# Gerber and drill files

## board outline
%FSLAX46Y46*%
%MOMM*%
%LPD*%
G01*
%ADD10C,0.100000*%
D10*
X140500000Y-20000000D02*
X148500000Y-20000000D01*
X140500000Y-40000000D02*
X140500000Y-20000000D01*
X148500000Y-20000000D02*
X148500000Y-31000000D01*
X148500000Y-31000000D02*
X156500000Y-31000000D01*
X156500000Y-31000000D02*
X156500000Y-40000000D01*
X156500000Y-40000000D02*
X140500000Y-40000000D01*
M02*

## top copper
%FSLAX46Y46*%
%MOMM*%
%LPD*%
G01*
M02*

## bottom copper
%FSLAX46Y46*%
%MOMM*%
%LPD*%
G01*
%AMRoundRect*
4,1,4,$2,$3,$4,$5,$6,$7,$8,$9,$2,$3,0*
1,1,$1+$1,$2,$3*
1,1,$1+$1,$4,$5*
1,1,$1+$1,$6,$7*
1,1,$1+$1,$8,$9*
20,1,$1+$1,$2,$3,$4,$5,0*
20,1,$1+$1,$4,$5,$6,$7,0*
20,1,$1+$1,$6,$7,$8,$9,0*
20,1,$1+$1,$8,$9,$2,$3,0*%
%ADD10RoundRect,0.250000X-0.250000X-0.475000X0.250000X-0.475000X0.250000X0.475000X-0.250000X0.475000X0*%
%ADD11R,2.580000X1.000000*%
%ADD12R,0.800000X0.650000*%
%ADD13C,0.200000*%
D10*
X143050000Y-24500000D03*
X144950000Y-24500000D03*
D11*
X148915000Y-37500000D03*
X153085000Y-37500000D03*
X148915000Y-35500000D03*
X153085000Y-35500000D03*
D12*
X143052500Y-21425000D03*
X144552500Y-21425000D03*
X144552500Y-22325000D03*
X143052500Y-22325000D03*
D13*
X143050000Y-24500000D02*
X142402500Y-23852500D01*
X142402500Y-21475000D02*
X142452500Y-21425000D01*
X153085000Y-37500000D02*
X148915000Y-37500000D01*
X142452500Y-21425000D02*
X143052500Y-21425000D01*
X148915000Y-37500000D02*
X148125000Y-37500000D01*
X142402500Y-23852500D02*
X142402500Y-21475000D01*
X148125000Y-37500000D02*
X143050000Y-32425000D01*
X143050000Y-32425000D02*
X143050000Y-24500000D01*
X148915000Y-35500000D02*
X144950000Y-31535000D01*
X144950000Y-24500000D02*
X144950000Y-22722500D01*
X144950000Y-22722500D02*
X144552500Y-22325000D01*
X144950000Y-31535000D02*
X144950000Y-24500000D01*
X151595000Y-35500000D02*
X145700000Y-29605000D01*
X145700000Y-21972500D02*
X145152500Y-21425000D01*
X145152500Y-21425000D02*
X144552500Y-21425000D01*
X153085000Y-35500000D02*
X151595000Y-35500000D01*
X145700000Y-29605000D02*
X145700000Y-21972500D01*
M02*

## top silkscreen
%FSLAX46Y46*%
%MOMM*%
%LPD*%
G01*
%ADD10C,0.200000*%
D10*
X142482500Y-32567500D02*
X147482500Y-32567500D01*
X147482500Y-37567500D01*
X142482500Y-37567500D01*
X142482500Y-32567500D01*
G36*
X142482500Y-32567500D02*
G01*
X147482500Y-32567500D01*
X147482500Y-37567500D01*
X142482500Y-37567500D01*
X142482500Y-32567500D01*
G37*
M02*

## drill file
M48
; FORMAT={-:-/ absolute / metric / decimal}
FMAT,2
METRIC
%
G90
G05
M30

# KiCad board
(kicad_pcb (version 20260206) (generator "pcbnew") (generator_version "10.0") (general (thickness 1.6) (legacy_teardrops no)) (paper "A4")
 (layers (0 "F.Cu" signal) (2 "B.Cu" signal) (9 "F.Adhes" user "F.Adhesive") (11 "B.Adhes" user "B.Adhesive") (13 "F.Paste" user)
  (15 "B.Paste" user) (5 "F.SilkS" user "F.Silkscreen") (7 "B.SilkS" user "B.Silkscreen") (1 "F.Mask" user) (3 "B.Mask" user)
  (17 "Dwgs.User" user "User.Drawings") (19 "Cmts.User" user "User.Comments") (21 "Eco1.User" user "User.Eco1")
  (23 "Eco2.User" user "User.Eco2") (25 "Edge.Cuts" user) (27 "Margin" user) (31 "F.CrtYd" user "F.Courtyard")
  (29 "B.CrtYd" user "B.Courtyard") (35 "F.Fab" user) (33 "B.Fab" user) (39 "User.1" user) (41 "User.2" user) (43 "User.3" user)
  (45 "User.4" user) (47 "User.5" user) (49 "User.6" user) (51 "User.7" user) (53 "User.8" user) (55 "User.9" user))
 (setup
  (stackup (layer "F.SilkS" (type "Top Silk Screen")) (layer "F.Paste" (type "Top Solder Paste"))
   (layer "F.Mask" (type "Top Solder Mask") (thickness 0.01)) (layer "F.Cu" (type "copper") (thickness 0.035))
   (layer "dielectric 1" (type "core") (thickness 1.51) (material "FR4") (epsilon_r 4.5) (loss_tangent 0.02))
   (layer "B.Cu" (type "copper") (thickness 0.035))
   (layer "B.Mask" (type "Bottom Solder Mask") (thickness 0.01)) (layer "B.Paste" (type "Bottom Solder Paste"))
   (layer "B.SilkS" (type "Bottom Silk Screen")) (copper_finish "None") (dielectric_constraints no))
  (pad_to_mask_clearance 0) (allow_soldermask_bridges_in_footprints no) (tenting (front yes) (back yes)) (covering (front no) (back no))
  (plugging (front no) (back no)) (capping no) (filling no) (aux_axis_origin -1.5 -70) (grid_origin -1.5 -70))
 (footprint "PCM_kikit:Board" (layer "F.Cu") (at 140.5 20)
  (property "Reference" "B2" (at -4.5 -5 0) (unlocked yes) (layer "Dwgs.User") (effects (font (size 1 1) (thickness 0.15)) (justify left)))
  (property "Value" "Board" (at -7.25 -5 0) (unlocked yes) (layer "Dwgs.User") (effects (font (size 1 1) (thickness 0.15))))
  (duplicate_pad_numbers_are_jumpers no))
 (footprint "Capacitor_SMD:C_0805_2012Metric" (layer "B.Cu") (at 144 24.5)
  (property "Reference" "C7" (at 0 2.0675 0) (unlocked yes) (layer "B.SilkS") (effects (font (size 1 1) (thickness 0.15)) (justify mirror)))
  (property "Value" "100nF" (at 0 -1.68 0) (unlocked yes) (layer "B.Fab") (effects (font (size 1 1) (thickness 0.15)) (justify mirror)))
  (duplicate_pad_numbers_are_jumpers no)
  (pad "1" smd roundrect (at -0.95 0) (size 1 1.45) (layers "B.Cu" "B.Mask" "B.Paste") (roundrect_rratio 0.25) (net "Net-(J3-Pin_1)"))
  (pad "2" smd roundrect (at 0.95 0) (size 1 1.45) (layers "B.Cu" "B.Mask" "B.Paste") (roundrect_rratio 0.25) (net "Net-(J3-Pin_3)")))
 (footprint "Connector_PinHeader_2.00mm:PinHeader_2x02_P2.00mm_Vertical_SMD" (layer "B.Cu") (at 151 36.5)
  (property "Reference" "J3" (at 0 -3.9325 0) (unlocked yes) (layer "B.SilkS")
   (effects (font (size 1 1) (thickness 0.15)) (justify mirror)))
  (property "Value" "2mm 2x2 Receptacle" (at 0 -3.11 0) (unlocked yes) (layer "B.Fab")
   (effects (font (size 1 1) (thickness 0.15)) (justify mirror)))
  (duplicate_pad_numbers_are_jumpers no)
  (pad "1" smd rect (at -2.085 1) (size 2.58 1) (layers "B.Cu" "B.Mask" "B.Paste") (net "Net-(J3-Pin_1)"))
  (pad "2" smd rect (at 2.085 1) (size 2.58 1) (layers "B.Cu" "B.Mask" "B.Paste") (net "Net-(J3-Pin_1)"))
  (pad "3" smd rect (at -2.085 -1) (size 2.58 1) (layers "B.Cu" "B.Mask" "B.Paste") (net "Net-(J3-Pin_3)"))
  (pad "4" smd rect (at 2.085 -1) (size 2.58 1) (layers "B.Cu" "B.Mask" "B.Paste") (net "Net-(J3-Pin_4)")))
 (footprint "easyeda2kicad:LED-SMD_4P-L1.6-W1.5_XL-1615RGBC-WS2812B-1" (layer "B.Cu") (at 143.8025 21.875)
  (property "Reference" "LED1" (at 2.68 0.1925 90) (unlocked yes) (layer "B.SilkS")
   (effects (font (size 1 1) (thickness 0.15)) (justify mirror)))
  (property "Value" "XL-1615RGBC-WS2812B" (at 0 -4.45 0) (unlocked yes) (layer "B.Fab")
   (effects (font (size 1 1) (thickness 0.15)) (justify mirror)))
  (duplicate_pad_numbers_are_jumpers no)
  (pad "1" smd rect (at -0.75 -0.45 180) (size 0.8 0.65) (layers "B.Cu" "B.Mask" "B.Paste") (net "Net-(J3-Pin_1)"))
  (pad "2" smd rect (at 0.75 -0.45 180) (size 0.8 0.65) (layers "B.Cu" "B.Mask" "B.Paste") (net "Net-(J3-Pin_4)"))
  (pad "3" smd rect (at 0.75 0.45 180) (size 0.8 0.65) (layers "B.Cu" "B.Mask" "B.Paste") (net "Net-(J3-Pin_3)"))
  (pad "4" smd rect (at -0.75 0.45 180) (size 0.8 0.65) (layers "B.Cu" "B.Mask" "B.Paste") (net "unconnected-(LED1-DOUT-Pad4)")))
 (gr_rect (start 142.4825 32.5675) (end 147.4825 37.5675) (stroke (width 0.2) (type solid)) (fill yes) (layer "F.SilkS"))
 (gr_line (start 140.5 20) (end 148.5 20) (stroke (width 0.1) (type default)) (layer "Edge.Cuts"))
 (gr_line (start 140.5 40) (end 140.5 20) (stroke (width 0.1) (type default)) (layer "Edge.Cuts"))
 (gr_line (start 148.5 20) (end 148.5 31) (stroke (width 0.1) (type default)) (layer "Edge.Cuts"))
 (gr_line (start 148.5 31) (end 156.5 31) (stroke (width 0.1) (type default)) (layer "Edge.Cuts"))
 (gr_line (start 156.5 31) (end 156.5 40) (stroke (width 0.1) (type default)) (layer "Edge.Cuts"))
 (gr_line (start 156.5 40) (end 140.5 40) (stroke (width 0.1) (type default)) (layer "Edge.Cuts"))
 (segment (start 143.05 24.5) (end 142.4025 23.8525) (width 0.2) (layer "B.Cu") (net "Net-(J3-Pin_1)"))
 (segment (start 142.4025 21.475) (end 142.4525 21.425) (width 0.2) (layer "B.Cu") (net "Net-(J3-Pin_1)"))
 (segment (start 153.085 37.5) (end 148.915 37.5) (width 0.2) (layer "B.Cu") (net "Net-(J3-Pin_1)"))
 (segment (start 142.4525 21.425) (end 143.0525 21.425) (width 0.2) (layer "B.Cu") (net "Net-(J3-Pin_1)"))
 (segment (start 148.915 37.5) (end 148.125 37.5) (width 0.2) (layer "B.Cu") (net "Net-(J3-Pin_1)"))
 (segment (start 142.4025 23.8525) (end 142.4025 21.475) (width 0.2) (layer "B.Cu") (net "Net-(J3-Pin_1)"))
 (segment (start 148.125 37.5) (end 143.05 32.425) (width 0.2) (layer "B.Cu") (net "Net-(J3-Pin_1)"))
 (segment (start 143.05 32.425) (end 143.05 24.5) (width 0.2) (layer "B.Cu") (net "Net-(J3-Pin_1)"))
 (segment (start 148.915 35.5) (end 144.95 31.535) (width 0.2) (layer "B.Cu") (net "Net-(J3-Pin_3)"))
 (segment (start 144.95 24.5) (end 144.95 22.7225) (width 0.2) (layer "B.Cu") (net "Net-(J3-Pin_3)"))
 (segment (start 144.95 22.7225) (end 144.5525 22.325) (width 0.2) (layer "B.Cu") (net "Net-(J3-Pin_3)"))
 (segment (start 144.95 31.535) (end 144.95 24.5) (width 0.2) (layer "B.Cu") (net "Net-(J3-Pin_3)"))
 (segment (start 151.595 35.5) (end 145.7 29.605) (width 0.2) (layer "B.Cu") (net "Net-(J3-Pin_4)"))
 (segment (start 145.7 21.9725) (end 145.1525 21.425) (width 0.2) (layer "B.Cu") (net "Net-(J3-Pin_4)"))
 (segment (start 145.1525 21.425) (end 144.5525 21.425) (width 0.2) (layer "B.Cu") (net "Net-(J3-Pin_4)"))
 (segment (start 153.085 35.5) (end 151.595 35.5) (width 0.2) (layer "B.Cu") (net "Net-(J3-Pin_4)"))
 (segment (start 145.7 29.605) (end 145.7 21.9725) (width 0.2) (layer "B.Cu") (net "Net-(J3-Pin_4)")))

